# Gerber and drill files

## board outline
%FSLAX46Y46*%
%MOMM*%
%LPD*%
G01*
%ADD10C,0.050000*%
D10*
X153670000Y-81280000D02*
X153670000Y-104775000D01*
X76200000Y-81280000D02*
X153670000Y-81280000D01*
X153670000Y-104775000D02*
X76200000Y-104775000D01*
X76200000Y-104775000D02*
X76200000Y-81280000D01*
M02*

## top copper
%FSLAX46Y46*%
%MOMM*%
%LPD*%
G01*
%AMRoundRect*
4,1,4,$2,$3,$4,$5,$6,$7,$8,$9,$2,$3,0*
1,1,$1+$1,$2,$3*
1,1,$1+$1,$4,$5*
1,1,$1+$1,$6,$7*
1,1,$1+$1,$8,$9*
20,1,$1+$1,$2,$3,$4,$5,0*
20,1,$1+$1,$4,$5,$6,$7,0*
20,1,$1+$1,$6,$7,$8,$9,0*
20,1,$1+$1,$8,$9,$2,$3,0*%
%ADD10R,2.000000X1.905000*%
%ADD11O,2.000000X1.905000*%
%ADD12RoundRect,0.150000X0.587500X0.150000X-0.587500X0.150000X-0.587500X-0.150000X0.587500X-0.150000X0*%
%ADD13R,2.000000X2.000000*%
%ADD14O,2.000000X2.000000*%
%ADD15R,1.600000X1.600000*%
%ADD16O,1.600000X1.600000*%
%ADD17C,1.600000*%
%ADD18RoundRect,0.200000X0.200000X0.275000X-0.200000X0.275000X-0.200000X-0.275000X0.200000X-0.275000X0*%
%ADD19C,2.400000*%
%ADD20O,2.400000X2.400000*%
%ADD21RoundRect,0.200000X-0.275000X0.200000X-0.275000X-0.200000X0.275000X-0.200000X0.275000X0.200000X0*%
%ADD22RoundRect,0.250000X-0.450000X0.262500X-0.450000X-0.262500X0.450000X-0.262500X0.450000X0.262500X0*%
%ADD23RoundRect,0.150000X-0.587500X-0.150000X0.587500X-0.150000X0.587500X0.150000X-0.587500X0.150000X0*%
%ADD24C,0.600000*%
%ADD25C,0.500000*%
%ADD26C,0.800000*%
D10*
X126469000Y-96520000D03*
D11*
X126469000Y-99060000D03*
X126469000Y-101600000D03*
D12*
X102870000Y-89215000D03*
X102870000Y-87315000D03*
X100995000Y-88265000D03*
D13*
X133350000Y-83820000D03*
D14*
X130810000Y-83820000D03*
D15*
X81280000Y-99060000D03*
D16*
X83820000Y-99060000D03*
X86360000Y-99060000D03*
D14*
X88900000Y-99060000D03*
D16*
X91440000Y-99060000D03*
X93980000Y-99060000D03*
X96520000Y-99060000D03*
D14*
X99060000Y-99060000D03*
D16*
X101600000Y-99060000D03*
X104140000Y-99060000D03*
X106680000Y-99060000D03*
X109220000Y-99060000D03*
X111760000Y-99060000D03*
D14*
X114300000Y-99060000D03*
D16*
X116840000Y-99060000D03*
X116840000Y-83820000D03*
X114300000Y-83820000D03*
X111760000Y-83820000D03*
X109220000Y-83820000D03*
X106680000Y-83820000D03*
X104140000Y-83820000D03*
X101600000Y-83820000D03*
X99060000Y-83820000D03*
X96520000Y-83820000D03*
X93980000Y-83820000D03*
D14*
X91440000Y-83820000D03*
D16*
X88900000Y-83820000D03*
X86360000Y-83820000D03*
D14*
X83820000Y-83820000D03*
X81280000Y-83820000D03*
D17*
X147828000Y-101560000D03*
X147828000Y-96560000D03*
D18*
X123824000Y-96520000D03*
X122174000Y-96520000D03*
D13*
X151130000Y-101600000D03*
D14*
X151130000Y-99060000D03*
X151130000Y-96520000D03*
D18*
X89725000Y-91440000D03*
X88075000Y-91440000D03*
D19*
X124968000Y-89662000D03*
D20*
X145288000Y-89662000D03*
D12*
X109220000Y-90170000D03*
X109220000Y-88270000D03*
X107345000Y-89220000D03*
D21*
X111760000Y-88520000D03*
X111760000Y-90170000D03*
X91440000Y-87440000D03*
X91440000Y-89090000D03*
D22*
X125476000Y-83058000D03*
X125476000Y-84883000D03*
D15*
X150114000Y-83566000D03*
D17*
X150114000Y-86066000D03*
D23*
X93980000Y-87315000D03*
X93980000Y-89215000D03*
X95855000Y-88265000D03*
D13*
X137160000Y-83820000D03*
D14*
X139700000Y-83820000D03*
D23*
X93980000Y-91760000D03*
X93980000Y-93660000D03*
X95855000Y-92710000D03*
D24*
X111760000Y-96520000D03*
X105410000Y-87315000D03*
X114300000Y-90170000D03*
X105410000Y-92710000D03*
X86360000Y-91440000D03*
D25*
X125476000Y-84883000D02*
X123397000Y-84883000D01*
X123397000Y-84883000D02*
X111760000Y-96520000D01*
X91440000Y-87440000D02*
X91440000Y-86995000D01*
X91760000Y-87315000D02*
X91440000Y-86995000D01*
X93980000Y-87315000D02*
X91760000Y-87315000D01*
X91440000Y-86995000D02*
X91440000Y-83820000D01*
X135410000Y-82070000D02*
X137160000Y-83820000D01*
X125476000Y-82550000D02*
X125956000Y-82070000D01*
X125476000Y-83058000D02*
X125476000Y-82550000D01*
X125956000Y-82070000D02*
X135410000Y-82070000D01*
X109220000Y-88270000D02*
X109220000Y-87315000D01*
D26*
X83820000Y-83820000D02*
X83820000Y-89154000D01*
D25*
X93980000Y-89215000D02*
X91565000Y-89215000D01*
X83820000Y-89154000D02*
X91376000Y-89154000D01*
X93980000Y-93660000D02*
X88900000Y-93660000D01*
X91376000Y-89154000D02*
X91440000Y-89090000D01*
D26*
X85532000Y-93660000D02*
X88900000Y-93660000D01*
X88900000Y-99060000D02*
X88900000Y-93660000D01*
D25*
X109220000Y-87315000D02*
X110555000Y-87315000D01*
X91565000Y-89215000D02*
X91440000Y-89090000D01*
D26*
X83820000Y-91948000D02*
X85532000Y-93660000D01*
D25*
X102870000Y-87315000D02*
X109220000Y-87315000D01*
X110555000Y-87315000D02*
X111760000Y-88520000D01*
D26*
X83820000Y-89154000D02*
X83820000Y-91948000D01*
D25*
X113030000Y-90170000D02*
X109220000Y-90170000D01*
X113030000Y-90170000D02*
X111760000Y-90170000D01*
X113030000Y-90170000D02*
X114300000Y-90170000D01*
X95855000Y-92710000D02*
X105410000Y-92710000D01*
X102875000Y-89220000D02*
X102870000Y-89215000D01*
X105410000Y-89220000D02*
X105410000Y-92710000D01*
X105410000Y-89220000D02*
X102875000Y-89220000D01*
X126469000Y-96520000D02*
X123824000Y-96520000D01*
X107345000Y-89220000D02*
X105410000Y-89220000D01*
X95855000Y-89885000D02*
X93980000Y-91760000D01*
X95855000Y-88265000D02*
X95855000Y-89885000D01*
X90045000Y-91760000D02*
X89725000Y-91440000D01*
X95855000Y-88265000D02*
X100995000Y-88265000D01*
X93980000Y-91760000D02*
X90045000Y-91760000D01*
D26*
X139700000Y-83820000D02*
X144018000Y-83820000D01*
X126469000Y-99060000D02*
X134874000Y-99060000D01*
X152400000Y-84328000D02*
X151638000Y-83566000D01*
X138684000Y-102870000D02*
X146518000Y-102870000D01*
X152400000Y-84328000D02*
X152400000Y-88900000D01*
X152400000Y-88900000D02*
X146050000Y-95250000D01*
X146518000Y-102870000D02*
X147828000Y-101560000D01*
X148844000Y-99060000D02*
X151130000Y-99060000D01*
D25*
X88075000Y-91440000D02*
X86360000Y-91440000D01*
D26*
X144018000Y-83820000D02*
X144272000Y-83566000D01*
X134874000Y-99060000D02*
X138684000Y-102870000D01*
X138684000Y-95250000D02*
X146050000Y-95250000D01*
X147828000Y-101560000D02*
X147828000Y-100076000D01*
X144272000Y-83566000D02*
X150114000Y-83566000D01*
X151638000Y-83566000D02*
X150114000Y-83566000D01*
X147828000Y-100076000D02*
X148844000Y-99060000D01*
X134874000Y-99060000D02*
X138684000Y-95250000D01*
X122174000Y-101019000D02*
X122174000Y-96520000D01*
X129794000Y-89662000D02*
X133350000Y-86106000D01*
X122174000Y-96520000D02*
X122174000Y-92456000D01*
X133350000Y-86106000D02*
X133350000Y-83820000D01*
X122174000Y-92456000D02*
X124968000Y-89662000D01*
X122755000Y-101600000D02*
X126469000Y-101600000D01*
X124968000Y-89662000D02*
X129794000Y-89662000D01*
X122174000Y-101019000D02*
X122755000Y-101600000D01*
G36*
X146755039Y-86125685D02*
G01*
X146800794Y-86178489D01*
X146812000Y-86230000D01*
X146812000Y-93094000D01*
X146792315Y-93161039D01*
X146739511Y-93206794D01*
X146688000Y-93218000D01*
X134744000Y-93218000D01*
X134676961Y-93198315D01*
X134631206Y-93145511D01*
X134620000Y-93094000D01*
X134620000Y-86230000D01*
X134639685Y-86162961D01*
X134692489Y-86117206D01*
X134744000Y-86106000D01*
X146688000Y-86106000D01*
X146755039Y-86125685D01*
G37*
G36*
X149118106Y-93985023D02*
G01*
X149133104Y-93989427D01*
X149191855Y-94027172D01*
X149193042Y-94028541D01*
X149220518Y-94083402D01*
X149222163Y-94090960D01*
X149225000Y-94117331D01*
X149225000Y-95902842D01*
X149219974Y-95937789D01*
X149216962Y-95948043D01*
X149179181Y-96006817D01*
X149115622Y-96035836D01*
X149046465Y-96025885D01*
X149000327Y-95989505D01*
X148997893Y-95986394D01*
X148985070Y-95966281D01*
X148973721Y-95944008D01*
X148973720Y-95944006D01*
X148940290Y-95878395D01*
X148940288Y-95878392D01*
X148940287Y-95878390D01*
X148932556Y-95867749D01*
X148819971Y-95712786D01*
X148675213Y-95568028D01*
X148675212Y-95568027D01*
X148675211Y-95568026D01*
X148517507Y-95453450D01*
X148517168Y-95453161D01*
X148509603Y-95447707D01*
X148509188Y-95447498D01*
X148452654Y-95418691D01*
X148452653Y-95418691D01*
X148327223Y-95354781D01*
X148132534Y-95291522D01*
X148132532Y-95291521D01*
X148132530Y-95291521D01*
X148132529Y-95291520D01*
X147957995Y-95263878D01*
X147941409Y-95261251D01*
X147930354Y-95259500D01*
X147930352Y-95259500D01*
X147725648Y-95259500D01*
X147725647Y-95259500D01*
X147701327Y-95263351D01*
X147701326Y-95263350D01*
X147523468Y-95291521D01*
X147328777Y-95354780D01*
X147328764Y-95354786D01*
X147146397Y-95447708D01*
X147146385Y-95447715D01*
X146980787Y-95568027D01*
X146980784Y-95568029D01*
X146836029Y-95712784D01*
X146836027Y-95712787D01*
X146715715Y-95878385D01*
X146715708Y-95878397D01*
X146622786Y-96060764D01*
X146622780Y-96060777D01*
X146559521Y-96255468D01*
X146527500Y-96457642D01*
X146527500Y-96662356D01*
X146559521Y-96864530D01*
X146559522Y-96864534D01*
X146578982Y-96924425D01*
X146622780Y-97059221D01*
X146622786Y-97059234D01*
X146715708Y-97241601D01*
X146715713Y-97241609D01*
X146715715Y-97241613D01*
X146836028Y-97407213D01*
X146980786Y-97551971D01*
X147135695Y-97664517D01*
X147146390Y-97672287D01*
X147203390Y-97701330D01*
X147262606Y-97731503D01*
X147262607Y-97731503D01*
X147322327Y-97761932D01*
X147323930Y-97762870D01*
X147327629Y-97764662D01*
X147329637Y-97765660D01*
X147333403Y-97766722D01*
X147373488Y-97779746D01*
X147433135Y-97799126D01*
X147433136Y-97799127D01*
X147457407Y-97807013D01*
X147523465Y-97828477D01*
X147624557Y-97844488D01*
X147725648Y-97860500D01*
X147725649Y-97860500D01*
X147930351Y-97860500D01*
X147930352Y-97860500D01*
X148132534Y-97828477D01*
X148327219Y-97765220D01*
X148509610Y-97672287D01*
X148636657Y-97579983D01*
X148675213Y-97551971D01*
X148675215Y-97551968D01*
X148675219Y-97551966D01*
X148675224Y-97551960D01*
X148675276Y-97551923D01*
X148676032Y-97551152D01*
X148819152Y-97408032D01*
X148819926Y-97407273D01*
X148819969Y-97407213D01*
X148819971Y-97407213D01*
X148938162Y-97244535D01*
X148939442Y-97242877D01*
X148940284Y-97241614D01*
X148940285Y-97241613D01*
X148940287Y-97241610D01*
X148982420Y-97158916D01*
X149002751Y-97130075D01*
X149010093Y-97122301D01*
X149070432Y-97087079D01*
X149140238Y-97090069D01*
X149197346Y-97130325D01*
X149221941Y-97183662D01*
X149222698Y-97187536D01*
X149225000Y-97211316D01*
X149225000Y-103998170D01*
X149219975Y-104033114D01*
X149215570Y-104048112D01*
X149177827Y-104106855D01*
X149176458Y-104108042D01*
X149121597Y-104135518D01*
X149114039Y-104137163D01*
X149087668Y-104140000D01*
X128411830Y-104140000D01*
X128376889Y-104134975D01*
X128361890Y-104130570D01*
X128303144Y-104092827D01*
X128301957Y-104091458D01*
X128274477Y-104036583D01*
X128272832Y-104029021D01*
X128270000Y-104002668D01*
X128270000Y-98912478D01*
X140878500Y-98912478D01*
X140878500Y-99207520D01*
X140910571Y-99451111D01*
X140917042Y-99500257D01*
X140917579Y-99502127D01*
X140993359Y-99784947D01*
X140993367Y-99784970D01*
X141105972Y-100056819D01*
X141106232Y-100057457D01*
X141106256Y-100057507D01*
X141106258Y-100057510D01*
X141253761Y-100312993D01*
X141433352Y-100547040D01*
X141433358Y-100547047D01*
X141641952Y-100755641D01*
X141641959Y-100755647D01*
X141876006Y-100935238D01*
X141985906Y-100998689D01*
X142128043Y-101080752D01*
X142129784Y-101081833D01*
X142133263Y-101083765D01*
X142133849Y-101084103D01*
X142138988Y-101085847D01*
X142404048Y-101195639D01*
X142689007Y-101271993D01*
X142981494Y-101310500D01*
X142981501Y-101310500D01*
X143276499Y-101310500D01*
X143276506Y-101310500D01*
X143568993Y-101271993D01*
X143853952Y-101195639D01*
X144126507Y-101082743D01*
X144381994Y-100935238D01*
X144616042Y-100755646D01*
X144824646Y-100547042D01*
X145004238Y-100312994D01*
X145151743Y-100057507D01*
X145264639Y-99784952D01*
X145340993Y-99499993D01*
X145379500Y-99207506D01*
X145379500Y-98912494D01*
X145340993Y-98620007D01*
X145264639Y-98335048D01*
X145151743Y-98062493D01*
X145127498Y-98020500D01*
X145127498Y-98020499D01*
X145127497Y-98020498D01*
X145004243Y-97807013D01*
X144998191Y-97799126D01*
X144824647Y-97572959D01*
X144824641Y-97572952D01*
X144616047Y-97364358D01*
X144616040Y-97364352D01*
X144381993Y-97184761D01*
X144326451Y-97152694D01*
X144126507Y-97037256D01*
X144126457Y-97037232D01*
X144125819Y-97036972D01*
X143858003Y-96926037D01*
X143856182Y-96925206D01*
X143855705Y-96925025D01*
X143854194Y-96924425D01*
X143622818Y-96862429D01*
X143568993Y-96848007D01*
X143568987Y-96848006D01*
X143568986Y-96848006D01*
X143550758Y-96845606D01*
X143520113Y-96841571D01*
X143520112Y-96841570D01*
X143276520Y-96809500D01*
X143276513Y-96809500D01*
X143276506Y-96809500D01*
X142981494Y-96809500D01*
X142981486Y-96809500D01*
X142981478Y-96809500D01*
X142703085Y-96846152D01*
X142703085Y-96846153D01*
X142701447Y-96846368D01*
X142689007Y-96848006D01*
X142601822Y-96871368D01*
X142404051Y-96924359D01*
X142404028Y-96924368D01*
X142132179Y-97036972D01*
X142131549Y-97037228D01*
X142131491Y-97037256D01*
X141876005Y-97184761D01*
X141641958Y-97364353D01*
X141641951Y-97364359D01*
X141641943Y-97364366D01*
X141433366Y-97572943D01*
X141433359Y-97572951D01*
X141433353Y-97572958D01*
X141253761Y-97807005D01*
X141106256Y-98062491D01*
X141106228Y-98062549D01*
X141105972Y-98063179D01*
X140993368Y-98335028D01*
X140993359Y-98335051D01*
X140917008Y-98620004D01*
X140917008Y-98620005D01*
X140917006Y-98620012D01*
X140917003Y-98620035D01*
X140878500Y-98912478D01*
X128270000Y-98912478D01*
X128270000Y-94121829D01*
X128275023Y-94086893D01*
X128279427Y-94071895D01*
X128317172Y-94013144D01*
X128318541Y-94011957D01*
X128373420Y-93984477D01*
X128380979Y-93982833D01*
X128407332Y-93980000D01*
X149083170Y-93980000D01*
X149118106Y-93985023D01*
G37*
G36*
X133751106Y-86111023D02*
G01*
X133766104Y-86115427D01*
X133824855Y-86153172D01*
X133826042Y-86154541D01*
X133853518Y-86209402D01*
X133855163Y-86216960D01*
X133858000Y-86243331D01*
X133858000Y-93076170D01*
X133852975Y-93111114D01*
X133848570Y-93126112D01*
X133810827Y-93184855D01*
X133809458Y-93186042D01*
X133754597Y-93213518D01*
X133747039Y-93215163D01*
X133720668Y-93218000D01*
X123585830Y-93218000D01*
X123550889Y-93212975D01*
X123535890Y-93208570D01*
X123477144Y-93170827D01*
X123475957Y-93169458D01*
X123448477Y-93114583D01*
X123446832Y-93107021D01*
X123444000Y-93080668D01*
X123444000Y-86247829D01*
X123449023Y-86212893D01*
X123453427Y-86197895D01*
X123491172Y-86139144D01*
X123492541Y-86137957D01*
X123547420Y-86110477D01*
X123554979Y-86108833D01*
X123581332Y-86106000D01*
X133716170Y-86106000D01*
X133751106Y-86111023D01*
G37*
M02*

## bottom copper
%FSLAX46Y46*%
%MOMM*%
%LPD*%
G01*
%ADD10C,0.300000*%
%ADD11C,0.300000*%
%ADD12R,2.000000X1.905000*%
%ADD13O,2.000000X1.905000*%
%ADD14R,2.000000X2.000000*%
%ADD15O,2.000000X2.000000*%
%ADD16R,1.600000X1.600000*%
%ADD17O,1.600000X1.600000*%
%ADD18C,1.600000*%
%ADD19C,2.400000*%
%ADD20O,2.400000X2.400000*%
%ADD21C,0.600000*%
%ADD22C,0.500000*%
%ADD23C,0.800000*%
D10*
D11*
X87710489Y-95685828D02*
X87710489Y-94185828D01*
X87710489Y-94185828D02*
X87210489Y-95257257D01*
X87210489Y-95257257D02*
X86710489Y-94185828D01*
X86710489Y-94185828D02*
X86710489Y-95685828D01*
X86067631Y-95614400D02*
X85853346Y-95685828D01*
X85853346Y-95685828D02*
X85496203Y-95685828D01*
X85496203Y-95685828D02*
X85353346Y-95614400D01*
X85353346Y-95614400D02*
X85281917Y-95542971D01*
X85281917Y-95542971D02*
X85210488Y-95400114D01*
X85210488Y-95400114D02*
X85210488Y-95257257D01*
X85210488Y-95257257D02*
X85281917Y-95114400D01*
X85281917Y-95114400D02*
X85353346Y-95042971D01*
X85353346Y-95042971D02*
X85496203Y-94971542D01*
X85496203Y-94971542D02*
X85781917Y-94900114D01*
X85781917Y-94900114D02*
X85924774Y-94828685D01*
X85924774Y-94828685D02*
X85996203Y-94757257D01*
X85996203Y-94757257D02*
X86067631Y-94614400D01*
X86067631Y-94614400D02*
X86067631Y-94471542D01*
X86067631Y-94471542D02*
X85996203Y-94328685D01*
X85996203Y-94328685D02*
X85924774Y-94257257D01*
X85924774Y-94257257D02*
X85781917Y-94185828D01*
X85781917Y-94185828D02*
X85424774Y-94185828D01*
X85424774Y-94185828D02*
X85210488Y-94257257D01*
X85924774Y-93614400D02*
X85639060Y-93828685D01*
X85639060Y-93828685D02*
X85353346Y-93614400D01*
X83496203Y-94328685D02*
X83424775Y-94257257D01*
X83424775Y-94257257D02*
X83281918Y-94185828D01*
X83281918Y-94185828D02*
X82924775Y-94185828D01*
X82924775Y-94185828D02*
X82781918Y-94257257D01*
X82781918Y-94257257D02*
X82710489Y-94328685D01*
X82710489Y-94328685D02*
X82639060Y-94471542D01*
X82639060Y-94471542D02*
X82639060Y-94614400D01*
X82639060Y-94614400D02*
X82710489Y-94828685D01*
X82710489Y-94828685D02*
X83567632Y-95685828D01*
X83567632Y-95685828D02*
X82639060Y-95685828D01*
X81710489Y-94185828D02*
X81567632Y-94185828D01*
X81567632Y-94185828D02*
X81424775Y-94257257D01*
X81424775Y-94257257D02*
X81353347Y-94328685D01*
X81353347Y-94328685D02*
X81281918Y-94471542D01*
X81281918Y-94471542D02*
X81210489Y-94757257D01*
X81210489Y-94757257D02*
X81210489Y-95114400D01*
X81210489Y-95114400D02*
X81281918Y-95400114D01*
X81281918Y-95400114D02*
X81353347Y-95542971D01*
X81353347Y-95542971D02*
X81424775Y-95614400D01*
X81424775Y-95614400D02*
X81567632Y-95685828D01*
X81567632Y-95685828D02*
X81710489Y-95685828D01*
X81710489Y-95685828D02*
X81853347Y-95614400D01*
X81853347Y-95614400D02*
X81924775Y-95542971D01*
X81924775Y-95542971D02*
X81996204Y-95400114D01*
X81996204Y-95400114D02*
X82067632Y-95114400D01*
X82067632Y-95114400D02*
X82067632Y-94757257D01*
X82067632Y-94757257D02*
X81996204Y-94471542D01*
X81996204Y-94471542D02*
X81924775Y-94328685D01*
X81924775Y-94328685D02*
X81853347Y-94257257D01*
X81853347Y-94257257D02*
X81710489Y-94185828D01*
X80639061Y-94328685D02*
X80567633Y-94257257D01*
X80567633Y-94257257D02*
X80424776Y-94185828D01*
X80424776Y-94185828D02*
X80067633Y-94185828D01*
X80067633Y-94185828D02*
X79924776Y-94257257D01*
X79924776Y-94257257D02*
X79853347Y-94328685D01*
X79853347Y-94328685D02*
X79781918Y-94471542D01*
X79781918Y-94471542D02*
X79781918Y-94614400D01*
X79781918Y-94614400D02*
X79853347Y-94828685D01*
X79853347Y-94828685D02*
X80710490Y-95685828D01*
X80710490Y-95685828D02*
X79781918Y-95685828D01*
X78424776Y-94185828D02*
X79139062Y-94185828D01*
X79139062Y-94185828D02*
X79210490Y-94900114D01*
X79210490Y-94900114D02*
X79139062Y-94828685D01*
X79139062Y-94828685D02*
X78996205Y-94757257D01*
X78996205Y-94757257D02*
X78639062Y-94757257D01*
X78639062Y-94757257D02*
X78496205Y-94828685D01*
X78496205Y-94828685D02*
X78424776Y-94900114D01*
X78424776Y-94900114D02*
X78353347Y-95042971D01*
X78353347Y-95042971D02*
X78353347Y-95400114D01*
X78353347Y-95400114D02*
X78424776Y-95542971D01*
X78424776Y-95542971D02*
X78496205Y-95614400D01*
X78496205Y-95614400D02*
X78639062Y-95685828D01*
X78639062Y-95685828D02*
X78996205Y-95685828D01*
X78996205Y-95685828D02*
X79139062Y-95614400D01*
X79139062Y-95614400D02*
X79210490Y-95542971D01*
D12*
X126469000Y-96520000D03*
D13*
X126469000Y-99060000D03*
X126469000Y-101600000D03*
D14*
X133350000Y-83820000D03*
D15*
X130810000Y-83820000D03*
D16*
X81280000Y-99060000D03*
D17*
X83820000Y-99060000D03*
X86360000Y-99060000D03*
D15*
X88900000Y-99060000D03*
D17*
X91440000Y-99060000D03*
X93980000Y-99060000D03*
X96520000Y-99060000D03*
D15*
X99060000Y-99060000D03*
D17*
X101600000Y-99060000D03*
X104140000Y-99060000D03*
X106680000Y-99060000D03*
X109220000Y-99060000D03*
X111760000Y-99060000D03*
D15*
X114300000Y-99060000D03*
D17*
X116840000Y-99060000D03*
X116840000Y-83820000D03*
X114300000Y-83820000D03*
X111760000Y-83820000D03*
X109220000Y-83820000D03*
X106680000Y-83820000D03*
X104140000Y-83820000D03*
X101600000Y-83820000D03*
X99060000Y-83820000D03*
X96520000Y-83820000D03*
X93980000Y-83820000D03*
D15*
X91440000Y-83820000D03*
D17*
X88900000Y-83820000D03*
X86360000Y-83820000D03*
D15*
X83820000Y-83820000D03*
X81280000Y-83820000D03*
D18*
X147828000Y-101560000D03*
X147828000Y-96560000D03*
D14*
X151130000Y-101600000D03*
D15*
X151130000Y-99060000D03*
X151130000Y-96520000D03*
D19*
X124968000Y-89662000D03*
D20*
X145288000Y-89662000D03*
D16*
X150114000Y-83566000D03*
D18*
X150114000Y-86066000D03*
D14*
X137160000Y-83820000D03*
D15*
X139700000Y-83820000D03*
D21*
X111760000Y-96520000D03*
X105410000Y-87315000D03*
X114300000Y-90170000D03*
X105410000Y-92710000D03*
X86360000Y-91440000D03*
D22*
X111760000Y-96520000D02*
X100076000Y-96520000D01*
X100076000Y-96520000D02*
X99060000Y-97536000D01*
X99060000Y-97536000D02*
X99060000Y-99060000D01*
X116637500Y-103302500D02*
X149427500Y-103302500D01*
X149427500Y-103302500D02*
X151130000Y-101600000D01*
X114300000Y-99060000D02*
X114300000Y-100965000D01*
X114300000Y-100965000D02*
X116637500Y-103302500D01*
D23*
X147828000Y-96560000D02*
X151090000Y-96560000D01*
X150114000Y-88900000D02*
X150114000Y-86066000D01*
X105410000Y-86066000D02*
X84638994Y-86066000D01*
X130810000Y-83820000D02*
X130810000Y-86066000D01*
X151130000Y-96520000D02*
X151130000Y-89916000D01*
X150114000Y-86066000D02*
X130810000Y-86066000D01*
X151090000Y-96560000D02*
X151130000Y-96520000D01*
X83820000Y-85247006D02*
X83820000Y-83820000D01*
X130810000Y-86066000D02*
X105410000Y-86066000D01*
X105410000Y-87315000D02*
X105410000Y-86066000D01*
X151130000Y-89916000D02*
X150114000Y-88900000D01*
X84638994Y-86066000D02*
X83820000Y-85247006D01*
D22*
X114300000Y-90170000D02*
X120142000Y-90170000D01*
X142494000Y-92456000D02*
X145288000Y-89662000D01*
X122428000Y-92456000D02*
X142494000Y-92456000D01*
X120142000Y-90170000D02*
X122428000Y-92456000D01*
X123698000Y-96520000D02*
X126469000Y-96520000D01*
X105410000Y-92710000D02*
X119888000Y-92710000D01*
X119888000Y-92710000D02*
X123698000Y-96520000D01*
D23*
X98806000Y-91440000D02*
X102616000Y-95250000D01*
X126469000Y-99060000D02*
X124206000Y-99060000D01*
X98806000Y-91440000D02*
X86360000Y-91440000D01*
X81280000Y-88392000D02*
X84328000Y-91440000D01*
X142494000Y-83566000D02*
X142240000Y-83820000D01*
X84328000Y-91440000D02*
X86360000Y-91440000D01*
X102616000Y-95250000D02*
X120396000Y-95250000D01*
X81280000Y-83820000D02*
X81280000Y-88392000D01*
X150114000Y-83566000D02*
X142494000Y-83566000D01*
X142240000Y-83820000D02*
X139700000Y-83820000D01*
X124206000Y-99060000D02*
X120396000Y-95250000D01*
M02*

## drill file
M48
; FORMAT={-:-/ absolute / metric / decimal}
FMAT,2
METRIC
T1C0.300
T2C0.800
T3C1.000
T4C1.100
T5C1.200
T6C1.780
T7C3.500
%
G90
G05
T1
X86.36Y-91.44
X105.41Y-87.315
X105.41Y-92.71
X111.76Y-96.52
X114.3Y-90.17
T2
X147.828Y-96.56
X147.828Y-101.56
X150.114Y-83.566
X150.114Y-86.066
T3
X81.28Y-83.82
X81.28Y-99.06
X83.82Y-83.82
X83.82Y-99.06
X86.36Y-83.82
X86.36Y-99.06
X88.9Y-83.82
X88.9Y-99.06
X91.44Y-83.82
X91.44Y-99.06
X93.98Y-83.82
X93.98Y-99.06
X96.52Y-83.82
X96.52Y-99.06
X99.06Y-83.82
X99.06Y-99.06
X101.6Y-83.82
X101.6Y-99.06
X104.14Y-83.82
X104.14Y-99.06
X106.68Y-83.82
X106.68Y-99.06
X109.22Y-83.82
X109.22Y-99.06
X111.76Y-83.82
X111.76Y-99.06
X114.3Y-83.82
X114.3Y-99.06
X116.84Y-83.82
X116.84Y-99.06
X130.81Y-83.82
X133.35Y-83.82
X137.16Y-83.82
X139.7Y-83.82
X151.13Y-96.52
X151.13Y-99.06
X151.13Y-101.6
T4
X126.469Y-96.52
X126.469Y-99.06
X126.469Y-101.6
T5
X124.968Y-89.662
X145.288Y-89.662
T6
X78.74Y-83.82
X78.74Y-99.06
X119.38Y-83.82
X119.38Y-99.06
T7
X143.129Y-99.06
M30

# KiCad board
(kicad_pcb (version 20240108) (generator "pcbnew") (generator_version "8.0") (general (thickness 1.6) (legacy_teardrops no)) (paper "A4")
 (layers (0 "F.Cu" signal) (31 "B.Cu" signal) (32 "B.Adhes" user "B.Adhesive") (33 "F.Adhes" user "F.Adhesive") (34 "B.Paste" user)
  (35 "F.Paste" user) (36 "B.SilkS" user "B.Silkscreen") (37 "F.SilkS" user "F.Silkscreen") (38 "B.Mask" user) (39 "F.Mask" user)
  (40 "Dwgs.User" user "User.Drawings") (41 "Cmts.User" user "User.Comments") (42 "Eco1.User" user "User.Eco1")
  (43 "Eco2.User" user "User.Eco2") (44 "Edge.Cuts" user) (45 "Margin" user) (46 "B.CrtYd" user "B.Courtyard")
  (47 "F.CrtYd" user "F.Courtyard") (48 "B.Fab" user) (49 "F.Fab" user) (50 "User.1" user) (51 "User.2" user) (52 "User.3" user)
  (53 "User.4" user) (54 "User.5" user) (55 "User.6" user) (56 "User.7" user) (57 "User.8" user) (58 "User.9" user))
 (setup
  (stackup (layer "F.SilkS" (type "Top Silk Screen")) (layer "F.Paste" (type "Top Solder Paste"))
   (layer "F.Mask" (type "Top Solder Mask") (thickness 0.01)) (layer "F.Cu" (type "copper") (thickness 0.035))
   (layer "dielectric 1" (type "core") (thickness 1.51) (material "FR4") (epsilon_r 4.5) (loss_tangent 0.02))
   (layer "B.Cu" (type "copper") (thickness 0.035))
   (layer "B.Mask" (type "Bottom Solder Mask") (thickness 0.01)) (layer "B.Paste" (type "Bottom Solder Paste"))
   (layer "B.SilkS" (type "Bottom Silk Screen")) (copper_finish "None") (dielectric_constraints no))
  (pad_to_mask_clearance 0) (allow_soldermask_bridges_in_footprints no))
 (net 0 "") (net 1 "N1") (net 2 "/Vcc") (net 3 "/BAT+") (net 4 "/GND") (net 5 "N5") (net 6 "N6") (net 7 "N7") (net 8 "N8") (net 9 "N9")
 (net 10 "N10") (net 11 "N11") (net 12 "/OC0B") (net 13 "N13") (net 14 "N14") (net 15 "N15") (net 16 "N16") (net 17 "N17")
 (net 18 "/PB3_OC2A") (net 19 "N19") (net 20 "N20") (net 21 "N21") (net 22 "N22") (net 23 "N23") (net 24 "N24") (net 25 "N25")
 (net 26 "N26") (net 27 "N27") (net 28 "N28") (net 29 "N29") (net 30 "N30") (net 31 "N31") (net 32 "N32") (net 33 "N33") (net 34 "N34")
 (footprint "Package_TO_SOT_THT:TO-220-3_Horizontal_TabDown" (layer "F.Cu") (at 126.469 96.52 -90)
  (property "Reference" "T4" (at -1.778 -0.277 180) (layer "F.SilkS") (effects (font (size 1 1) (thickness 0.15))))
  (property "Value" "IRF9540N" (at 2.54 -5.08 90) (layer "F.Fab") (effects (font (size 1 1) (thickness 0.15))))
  (pad "" np_thru_hole oval (at 2.54 -16.66 270) (size 3.5 3.5) (drill 3.5) (layers "*.Cu" "*.Mask"))
  (pad "1" thru_hole rect (at 0 0 270) (size 1.905 2) (drill 1.1) (layers "*.Cu" "*.Mask") (remove_unused_layers no) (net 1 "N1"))
  (pad "2" thru_hole oval (at 2.54 0 270) (size 1.905 2) (drill 1.1) (layers "*.Cu" "*.Mask") (remove_unused_layers no) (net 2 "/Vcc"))
  (pad "3" thru_hole oval (at 5.08 0 270) (size 1.905 2) (drill 1.1) (layers "*.Cu" "*.Mask") (remove_unused_layers no) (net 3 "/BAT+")))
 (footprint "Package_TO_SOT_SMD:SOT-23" (layer "F.Cu") (at 101.9325 88.265 180)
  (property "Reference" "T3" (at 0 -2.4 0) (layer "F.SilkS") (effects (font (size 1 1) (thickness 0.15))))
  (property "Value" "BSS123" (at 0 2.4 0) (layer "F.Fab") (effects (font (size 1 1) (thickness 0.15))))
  (pad "1" smd roundrect (at -0.9375 -0.95 180) (size 1.475 0.6) (layers "F.Cu" "F.Paste" "F.Mask") (roundrect_rratio 0.25) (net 1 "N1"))
  (pad "2" smd roundrect (at -0.9375 0.95 180) (size 1.475 0.6) (layers "F.Cu" "F.Paste" "F.Mask") (roundrect_rratio 0.25) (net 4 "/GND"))
  (pad "3" smd roundrect (at 0.9375 0 180) (size 1.475 0.6) (layers "F.Cu" "F.Paste" "F.Mask") (roundrect_rratio 0.25) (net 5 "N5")))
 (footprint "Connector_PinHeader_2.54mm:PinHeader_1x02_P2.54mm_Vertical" (layer "F.Cu") (at 133.35 83.82 -90)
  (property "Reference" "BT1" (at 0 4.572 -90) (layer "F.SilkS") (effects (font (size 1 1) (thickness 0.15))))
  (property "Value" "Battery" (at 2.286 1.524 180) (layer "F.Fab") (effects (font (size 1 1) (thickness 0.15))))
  (pad "1" thru_hole rect (at 0 0 270) (size 2 2) (drill 1) (layers "*.Cu" "*.Mask") (remove_unused_layers no) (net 3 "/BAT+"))
  (pad "2" thru_hole oval (at 0 2.54 270) (size 2 2) (drill 1) (layers "*.Cu" "*.Mask") (remove_unused_layers no) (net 4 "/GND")))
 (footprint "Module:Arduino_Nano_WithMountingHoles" (layer "F.Cu") (at 81.28 99.06 90)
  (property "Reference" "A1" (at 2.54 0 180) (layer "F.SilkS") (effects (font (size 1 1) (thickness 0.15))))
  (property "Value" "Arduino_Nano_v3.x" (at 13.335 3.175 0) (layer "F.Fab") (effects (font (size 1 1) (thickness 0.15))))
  (pad "" np_thru_hole circle (at 0 -2.54 90) (size 1.78 1.78) (drill 1.78) (layers "*.Cu" "*.Mask"))
  (pad "" np_thru_hole circle (at 0 38.1 90) (size 1.78 1.78) (drill 1.78) (layers "*.Cu" "*.Mask"))
  (pad "" np_thru_hole circle (at 15.24 -2.54 90) (size 1.78 1.78) (drill 1.78) (layers "*.Cu" "*.Mask"))
  (pad "" np_thru_hole circle (at 15.24 38.1 90) (size 1.78 1.78) (drill 1.78) (layers "*.Cu" "*.Mask"))
  (pad "1" thru_hole rect (at 0 0 90) (size 1.6 1.6) (drill 1) (layers "*.Cu" "*.Mask") (remove_unused_layers no) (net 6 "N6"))
  (pad "2" thru_hole oval (at 0 2.54 90) (size 1.6 1.6) (drill 1) (layers "*.Cu" "*.Mask") (remove_unused_layers no) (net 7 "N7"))
  (pad "3" thru_hole oval (at 0 5.08 90) (size 1.6 1.6) (drill 1) (layers "*.Cu" "*.Mask") (remove_unused_layers no) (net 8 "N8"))
  (pad "4" thru_hole oval (at 0 7.62 90) (size 2 2) (drill 1) (layers "*.Cu" "*.Mask") (remove_unused_layers no) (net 4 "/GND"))
  (pad "5" thru_hole oval (at 0 10.16 90) (size 1.6 1.6) (drill 1) (layers "*.Cu" "*.Mask") (remove_unused_layers no) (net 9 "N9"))
  (pad "6" thru_hole oval (at 0 12.7 90) (size 1.6 1.6) (drill 1) (layers "*.Cu" "*.Mask") (remove_unused_layers no) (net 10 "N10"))
  (pad "7" thru_hole oval (at 0 15.24 90) (size 1.6 1.6) (drill 1) (layers "*.Cu" "*.Mask") (remove_unused_layers no) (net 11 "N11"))
  (pad "8" thru_hole oval (at 0 17.78 90) (size 2 2) (drill 1) (layers "*.Cu" "*.Mask") (remove_unused_layers no) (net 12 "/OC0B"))
  (pad "9" thru_hole oval (at 0 20.32 90) (size 1.6 1.6) (drill 1) (layers "*.Cu" "*.Mask") (remove_unused_layers no) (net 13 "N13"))
  (pad "10" thru_hole oval (at 0 22.86 90) (size 1.6 1.6) (drill 1) (layers "*.Cu" "*.Mask") (remove_unused_layers no) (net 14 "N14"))
  (pad "11" thru_hole oval (at 0 25.4 90) (size 1.6 1.6) (drill 1) (layers "*.Cu" "*.Mask") (remove_unused_layers no) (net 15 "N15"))
  (pad "12" thru_hole oval (at 0 27.94 90) (size 1.6 1.6) (drill 1) (layers "*.Cu" "*.Mask") (remove_unused_layers no) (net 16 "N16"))
  (pad "13" thru_hole oval (at 0 30.48 90) (size 1.6 1.6) (drill 1) (layers "*.Cu" "*.Mask") (remove_unused_layers no) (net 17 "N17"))
  (pad "14" thru_hole oval (at 0 33.02 90) (size 2 2) (drill 1) (layers "*.Cu" "*.Mask") (remove_unused_layers no) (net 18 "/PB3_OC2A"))
  (pad "15" thru_hole oval (at 0 35.56 90) (size 1.6 1.6) (drill 1) (layers "*.Cu" "*.Mask") (remove_unused_layers no) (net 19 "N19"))
  (pad "16" thru_hole oval (at 15.24 35.56 90) (size 1.6 1.6) (drill 1) (layers "*.Cu" "*.Mask") (remove_unused_layers no) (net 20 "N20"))
  (pad "17" thru_hole oval (at 15.24 33.02 90) (size 1.6 1.6) (drill 1) (layers "*.Cu" "*.Mask") (remove_unused_layers no) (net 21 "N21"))
  (pad "18" thru_hole oval (at 15.24 30.48 90) (size 1.6 1.6) (drill 1) (layers "*.Cu" "*.Mask") (remove_unused_layers no) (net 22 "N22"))
  (pad "19" thru_hole oval (at 15.24 27.94 90) (size 1.6 1.6) (drill 1) (layers "*.Cu" "*.Mask") (remove_unused_layers no) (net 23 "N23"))
  (pad "20" thru_hole oval (at 15.24 25.4 90) (size 1.6 1.6) (drill 1) (layers "*.Cu" "*.Mask") (remove_unused_layers no) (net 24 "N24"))
  (pad "21" thru_hole oval (at 15.24 22.86 90) (size 1.6 1.6) (drill 1) (layers "*.Cu" "*.Mask") (remove_unused_layers no) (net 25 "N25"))
  (pad "22" thru_hole oval (at 15.24 20.32 90) (size 1.6 1.6) (drill 1) (layers "*.Cu" "*.Mask") (remove_unused_layers no) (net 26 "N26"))
  (pad "23" thru_hole oval (at 15.24 17.78 90) (size 1.6 1.6) (drill 1) (layers "*.Cu" "*.Mask") (remove_unused_layers no) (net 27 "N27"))
  (pad "24" thru_hole oval (at 15.24 15.24 90) (size 1.6 1.6) (drill 1) (layers "*.Cu" "*.Mask") (remove_unused_layers no) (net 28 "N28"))
  (pad "25" thru_hole oval (at 15.24 12.7 90) (size 1.6 1.6) (drill 1) (layers "*.Cu" "*.Mask") (remove_unused_layers no) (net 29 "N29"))
  (pad "26" thru_hole oval (at 15.24 10.16 90) (size 2 2) (drill 1) (layers "*.Cu" "*.Mask") (remove_unused_layers no) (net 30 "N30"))
  (pad "27" thru_hole oval (at 15.24 7.62 90) (size 1.6 1.6) (drill 1) (layers "*.Cu" "*.Mask") (remove_unused_layers no) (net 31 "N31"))
  (pad "28" thru_hole oval (at 15.24 5.08 90) (size 1.6 1.6) (drill 1) (layers "*.Cu" "*.Mask") (remove_unused_layers no) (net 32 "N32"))
  (pad "29" thru_hole oval (at 15.24 2.54 90) (size 2 2) (drill 1) (layers "*.Cu" "*.Mask") (remove_unused_layers no) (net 4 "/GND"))
  (pad "30" thru_hole oval (at 15.24 0 90) (size 2 2) (drill 1) (layers "*.Cu" "*.Mask") (remove_unused_layers no) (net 2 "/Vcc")))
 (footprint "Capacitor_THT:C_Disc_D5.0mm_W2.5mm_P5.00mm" (layer "F.Cu") (at 147.828 101.56 90)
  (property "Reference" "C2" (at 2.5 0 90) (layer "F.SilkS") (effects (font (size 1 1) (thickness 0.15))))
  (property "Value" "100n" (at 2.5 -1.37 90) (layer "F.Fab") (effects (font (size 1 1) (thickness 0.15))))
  (pad "1" thru_hole circle (at 0 0 90) (size 1.6 1.6) (drill 0.8) (layers "*.Cu" "*.Mask") (remove_unused_layers no) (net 2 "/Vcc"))
  (pad "2" thru_hole circle (at 5 0 90) (size 1.6 1.6) (drill 0.8) (layers "*.Cu" "*.Mask") (remove_unused_layers no) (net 4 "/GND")))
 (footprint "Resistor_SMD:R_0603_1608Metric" (layer "F.Cu") (at 122.999 96.52 180)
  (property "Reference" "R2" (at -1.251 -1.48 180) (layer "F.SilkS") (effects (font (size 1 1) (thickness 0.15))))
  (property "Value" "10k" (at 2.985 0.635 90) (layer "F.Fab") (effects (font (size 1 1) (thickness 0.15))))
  (pad "1" smd roundrect (at -0.825 0 180) (size 0.8 0.95) (layers "F.Cu" "F.Paste" "F.Mask") (roundrect_rratio 0.25) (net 1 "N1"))
  (pad "2" smd roundrect (at 0.825 0 180) (size 0.8 0.95) (layers "F.Cu" "F.Paste" "F.Mask") (roundrect_rratio 0.25) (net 3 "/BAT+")))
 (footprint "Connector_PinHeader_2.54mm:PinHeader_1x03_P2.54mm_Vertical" (layer "F.Cu") (at 151.13 101.6 180)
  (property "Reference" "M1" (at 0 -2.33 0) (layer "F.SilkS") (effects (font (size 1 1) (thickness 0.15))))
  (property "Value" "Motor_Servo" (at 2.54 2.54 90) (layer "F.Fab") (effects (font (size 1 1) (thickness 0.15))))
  (pad "1" thru_hole rect (at 0 0 180) (size 2 2) (drill 1) (layers "*.Cu" "*.Mask") (remove_unused_layers no) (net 18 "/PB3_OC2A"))
  (pad "2" thru_hole oval (at 0 2.54 180) (size 2 2) (drill 1) (layers "*.Cu" "*.Mask") (remove_unused_layers no) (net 2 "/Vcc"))
  (pad "3" thru_hole oval (at 0 5.08 180) (size 2 2) (drill 1) (layers "*.Cu" "*.Mask") (remove_unused_layers no) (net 4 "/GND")))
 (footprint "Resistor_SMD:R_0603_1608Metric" (layer "F.Cu") (at 88.9 91.44 180)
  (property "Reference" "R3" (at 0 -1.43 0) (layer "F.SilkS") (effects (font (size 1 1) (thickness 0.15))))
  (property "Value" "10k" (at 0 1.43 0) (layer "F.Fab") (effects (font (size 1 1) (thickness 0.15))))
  (pad "1" smd roundrect (at -0.825 0 180) (size 0.8 0.95) (layers "F.Cu" "F.Paste" "F.Mask") (roundrect_rratio 0.25) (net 5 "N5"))
  (pad "2" smd roundrect (at 0.825 0 180) (size 0.8 0.95) (layers "F.Cu" "F.Paste" "F.Mask") (roundrect_rratio 0.25) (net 2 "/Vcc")))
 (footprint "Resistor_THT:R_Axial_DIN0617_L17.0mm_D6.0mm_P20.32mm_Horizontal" (layer "F.Cu") (at 124.968 89.662)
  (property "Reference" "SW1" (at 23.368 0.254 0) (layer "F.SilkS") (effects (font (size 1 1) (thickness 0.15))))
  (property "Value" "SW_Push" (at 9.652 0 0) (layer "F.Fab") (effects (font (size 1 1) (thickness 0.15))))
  (pad "1" thru_hole circle (at 0 0) (size 2.4 2.4) (drill 1.2) (layers "*.Cu" "*.Mask") (remove_unused_layers no) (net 3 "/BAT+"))
  (pad "2" thru_hole oval (at 20.32 0) (size 2.4 2.4) (drill 1.2) (layers "*.Cu" "*.Mask") (remove_unused_layers no) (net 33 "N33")))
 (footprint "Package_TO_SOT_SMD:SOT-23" (layer "F.Cu") (at 108.2825 89.22 180)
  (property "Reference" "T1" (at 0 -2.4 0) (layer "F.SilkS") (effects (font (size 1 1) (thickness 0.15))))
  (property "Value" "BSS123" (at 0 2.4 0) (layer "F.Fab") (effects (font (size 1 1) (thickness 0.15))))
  (pad "1" smd roundrect (at -0.9375 -0.95 180) (size 1.475 0.6) (layers "F.Cu" "F.Paste" "F.Mask") (roundrect_rratio 0.25) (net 33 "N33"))
  (pad "2" smd roundrect (at -0.9375 0.95 180) (size 1.475 0.6) (layers "F.Cu" "F.Paste" "F.Mask") (roundrect_rratio 0.25) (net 4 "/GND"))
  (pad "3" smd roundrect (at 0.9375 0 180) (size 1.475 0.6) (layers "F.Cu" "F.Paste" "F.Mask") (roundrect_rratio 0.25) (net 1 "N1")))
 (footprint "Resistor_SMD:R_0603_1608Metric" (layer "F.Cu") (at 111.76 89.345 -90)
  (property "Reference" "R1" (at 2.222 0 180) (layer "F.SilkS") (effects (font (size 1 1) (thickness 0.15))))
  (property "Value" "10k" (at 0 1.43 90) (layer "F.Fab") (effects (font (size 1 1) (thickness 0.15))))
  (pad "1" smd roundrect (at -0.825 0 270) (size 0.8 0.95) (layers "F.Cu" "F.Paste" "F.Mask") (roundrect_rratio 0.25) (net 4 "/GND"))
  (pad "2" smd roundrect (at 0.825 0 270) (size 0.8 0.95) (layers "F.Cu" "F.Paste" "F.Mask") (roundrect_rratio 0.25) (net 33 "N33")))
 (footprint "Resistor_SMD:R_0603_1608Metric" (layer "F.Cu") (at 91.44 88.265 -90)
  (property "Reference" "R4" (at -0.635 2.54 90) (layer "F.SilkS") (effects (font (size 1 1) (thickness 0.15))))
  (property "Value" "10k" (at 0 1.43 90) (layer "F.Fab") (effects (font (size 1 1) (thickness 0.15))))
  (pad "1" smd roundrect (at -0.825 0 270) (size 0.8 0.95) (layers "F.Cu" "F.Paste" "F.Mask") (roundrect_rratio 0.25) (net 30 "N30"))
  (pad "2" smd roundrect (at 0.825 0 270) (size 0.8 0.95) (layers "F.Cu" "F.Paste" "F.Mask") (roundrect_rratio 0.25) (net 4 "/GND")))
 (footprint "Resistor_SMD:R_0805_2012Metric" (layer "F.Cu") (at 125.476 83.9705 -90)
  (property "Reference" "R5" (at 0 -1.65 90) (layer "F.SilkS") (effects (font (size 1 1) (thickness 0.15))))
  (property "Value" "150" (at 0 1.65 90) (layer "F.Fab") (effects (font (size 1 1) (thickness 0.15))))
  (pad "1" smd roundrect (at -0.9125 0 270) (size 1.025 1.4) (layers "F.Cu" "F.Paste" "F.Mask") (roundrect_rratio 0.243902) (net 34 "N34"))
  (pad "2" smd roundrect (at 0.9125 0 270) (size 1.025 1.4) (layers "F.Cu" "F.Paste" "F.Mask") (roundrect_rratio 0.243902) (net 12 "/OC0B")))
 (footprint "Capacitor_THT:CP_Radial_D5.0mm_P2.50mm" (layer "F.Cu") (at 150.114 83.566 -90)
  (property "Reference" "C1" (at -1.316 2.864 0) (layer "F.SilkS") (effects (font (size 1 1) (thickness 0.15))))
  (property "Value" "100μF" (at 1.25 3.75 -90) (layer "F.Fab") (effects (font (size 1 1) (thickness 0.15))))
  (pad "1" thru_hole rect (at 0 0 270) (size 1.6 1.6) (drill 0.8) (layers "*.Cu" "*.Mask") (remove_unused_layers no) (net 2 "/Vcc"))
  (pad "2" thru_hole circle (at 2.5 0 270) (size 1.6 1.6) (drill 0.8) (layers "*.Cu" "*.Mask") (remove_unused_layers no) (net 4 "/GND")))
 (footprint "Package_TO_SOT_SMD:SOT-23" (layer "F.Cu") (at 94.9175 88.265)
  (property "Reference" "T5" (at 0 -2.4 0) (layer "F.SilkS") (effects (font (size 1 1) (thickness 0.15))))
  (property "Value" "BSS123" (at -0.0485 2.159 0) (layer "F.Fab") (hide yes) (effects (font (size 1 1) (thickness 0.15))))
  (pad "1" smd roundrect (at -0.9375 -0.95) (size 1.475 0.6) (layers "F.Cu" "F.Paste" "F.Mask") (roundrect_rratio 0.25) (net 30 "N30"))
  (pad "2" smd roundrect (at -0.9375 0.95) (size 1.475 0.6) (layers "F.Cu" "F.Paste" "F.Mask") (roundrect_rratio 0.25) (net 4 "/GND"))
  (pad "3" smd roundrect (at 0.9375 0) (size 1.475 0.6) (layers "F.Cu" "F.Paste" "F.Mask") (roundrect_rratio 0.25) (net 5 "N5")))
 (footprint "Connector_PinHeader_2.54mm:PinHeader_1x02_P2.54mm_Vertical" (layer "F.Cu") (at 137.16 83.82 90)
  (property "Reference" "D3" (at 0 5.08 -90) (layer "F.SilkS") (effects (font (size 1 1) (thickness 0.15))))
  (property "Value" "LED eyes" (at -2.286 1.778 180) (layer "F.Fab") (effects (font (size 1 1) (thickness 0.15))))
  (pad "1" thru_hole rect (at 0 0 90) (size 2 2) (drill 1) (layers "*.Cu" "*.Mask") (remove_unused_layers no) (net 34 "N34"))
  (pad "2" thru_hole oval (at 0 2.54 90) (size 2 2) (drill 1) (layers "*.Cu" "*.Mask") (remove_unused_layers no) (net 2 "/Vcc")))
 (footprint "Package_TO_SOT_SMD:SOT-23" (layer "F.Cu") (at 94.9175 92.71)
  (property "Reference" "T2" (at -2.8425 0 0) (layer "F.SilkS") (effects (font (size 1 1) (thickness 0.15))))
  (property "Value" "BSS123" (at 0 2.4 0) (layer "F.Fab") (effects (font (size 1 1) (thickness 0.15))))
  (pad "1" smd roundrect (at -0.9375 -0.95) (size 1.475 0.6) (layers "F.Cu" "F.Paste" "F.Mask") (roundrect_rratio 0.25) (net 5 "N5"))
  (pad "2" smd roundrect (at -0.9375 0.95) (size 1.475 0.6) (layers "F.Cu" "F.Paste" "F.Mask") (roundrect_rratio 0.25) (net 4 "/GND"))
  (pad "3" smd roundrect (at 0.9375 0) (size 1.475 0.6) (layers "F.Cu" "F.Paste" "F.Mask") (roundrect_rratio 0.25) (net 1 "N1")))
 (gr_line (start 153.67 81.28) (end 153.67 104.775) (stroke (width 0.05) (type default)) (layer "Edge.Cuts"))
 (gr_line (start 76.2 81.28) (end 153.67 81.28) (stroke (width 0.05) (type default)) (layer "Edge.Cuts"))
 (gr_line (start 153.67 104.775) (end 76.2 104.775) (stroke (width 0.05) (type default)) (layer "Edge.Cuts"))
 (gr_line (start 76.2 104.775) (end 76.2 81.28) (stroke (width 0.05) (type default)) (layer "Edge.Cuts"))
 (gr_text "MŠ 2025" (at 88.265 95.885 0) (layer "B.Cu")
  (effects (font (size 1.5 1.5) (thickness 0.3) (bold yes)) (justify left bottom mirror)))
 (segment (start 125.476 84.883) (end 123.397 84.883) (width 0.5) (layer "F.Cu") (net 12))
 (segment (start 123.397 84.883) (end 111.76 96.52) (width 0.5) (layer "F.Cu") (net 12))
 (via (at 111.76 96.52) (size 0.6) (drill 0.3) (layers "F.Cu" "B.Cu") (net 12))
 (segment (start 111.76 96.52) (end 100.076 96.52) (width 0.5) (layer "B.Cu") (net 12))
 (segment (start 100.076 96.52) (end 99.06 97.536) (width 0.5) (layer "B.Cu") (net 12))
 (segment (start 99.06 97.536) (end 99.06 99.06) (width 0.5) (layer "B.Cu") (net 12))
 (segment (start 116.6375 103.3025) (end 149.4275 103.3025) (width 0.5) (layer "B.Cu") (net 18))
 (segment (start 149.4275 103.3025) (end 151.13 101.6) (width 0.5) (layer "B.Cu") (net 18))
 (segment (start 114.3 99.06) (end 114.3 100.965) (width 0.5) (layer "B.Cu") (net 18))
 (segment (start 114.3 100.965) (end 116.6375 103.3025) (width 0.5) (layer "B.Cu") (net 18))
 (segment (start 91.44 87.44) (end 91.44 86.995) (width 0.5) (layer "F.Cu") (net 30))
 (segment (start 91.76 87.315) (end 91.44 86.995) (width 0.5) (layer "F.Cu") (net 30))
 (segment (start 93.98 87.315) (end 91.76 87.315) (width 0.5) (layer "F.Cu") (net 30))
 (segment (start 91.44 86.995) (end 91.44 83.82) (width 0.5) (layer "F.Cu") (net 30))
 (segment (start 135.41 82.07) (end 137.16 83.82) (width 0.5) (layer "F.Cu") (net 34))
 (segment (start 125.476 82.55) (end 125.956 82.07) (width 0.5) (layer "F.Cu") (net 34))
 (segment (start 125.476 83.058) (end 125.476 82.55) (width 0.5) (layer "F.Cu") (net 34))
 (segment (start 125.956 82.07) (end 135.41 82.07) (width 0.5) (layer "F.Cu") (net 34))
 (segment (start 109.22 88.27) (end 109.22 87.315) (width 0.5) (layer "F.Cu") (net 4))
 (segment (start 83.82 83.82) (end 83.82 89.154) (width 0.8) (layer "F.Cu") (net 4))
 (segment (start 93.98 89.215) (end 91.565 89.215) (width 0.5) (layer "F.Cu") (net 4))
 (segment (start 83.82 89.154) (end 91.376 89.154) (width 0.5) (layer "F.Cu") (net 4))
 (segment (start 93.98 93.66) (end 88.9 93.66) (width 0.5) (layer "F.Cu") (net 4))
 (segment (start 91.376 89.154) (end 91.44 89.09) (width 0.5) (layer "F.Cu") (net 4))
 (segment (start 85.532 93.66) (end 88.9 93.66) (width 0.8) (layer "F.Cu") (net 4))
 (segment (start 88.9 99.06) (end 88.9 93.66) (width 0.8) (layer "F.Cu") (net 4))
 (segment (start 109.22 87.315) (end 110.555 87.315) (width 0.5) (layer "F.Cu") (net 4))
 (segment (start 91.565 89.215) (end 91.44 89.09) (width 0.5) (layer "F.Cu") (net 4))
 (segment (start 83.82 91.948) (end 85.532 93.66) (width 0.8) (layer "F.Cu") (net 4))
 (segment (start 102.87 87.315) (end 109.22 87.315) (width 0.5) (layer "F.Cu") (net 4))
 (segment (start 110.555 87.315) (end 111.76 88.52) (width 0.5) (layer "F.Cu") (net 4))
 (segment (start 83.82 89.154) (end 83.82 91.948) (width 0.8) (layer "F.Cu") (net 4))
 (via (at 105.41 87.315) (size 0.6) (drill 0.3) (layers "F.Cu" "B.Cu") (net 4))
 (segment (start 147.828 96.56) (end 151.09 96.56) (width 0.8) (layer "B.Cu") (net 4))
 (segment (start 150.114 88.9) (end 150.114 86.066) (width 0.8) (layer "B.Cu") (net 4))
 (segment (start 105.41 86.066) (end 84.638994 86.066) (width 0.8) (layer "B.Cu") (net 4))
 (segment (start 130.81 83.82) (end 130.81 86.066) (width 0.8) (layer "B.Cu") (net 4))
 (segment (start 151.13 96.52) (end 151.13 89.916) (width 0.8) (layer "B.Cu") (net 4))
 (segment (start 150.114 86.066) (end 130.81 86.066) (width 0.8) (layer "B.Cu") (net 4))
 (segment (start 151.09 96.56) (end 151.13 96.52) (width 0.8) (layer "B.Cu") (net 4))
 (segment (start 83.82 85.247006) (end 83.82 83.82) (width 0.8) (layer "B.Cu") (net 4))
 (segment (start 130.81 86.066) (end 105.41 86.066) (width 0.8) (layer "B.Cu") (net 4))
 (segment (start 105.41 87.315) (end 105.41 86.066) (width 0.8) (layer "B.Cu") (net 4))
 (segment (start 151.13 89.916) (end 150.114 88.9) (width 0.8) (layer "B.Cu") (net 4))
 (segment (start 84.638994 86.066) (end 83.82 85.247006) (width 0.8) (layer "B.Cu") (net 4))
 (segment (start 113.03 90.17) (end 109.22 90.17) (width 0.5) (layer "F.Cu") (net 33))
 (segment (start 113.03 90.17) (end 111.76 90.17) (width 0.5) (layer "F.Cu") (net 33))
 (segment (start 113.03 90.17) (end 114.3 90.17) (width 0.5) (layer "F.Cu") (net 33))
 (via (at 114.3 90.17) (size 0.6) (drill 0.3) (layers "F.Cu" "B.Cu") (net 33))
 (segment (start 114.3 90.17) (end 120.142 90.17) (width 0.5) (layer "B.Cu") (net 33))
 (segment (start 142.494 92.456) (end 145.288 89.662) (width 0.5) (layer "B.Cu") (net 33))
 (segment (start 122.428 92.456) (end 142.494 92.456) (width 0.5) (layer "B.Cu") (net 33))
 (segment (start 120.142 90.17) (end 122.428 92.456) (width 0.5) (layer "B.Cu") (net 33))
 (segment (start 95.855 92.71) (end 105.41 92.71) (width 0.5) (layer "F.Cu") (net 1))
 (segment (start 102.875 89.22) (end 102.87 89.215) (width 0.5) (layer "F.Cu") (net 1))
 (segment (start 105.41 89.22) (end 105.41 92.71) (width 0.5) (layer "F.Cu") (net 1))
 (segment (start 105.41 89.22) (end 102.875 89.22) (width 0.5) (layer "F.Cu") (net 1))
 (segment (start 126.469 96.52) (end 123.824 96.52) (width 0.5) (layer "F.Cu") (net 1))
 (segment (start 107.345 89.22) (end 105.41 89.22) (width 0.5) (layer "F.Cu") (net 1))
 (via (at 105.41 92.71) (size 0.6) (drill 0.3) (layers "F.Cu" "B.Cu") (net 1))
 (segment (start 123.698 96.52) (end 126.469 96.52) (width 0.5) (layer "B.Cu") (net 1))
 (segment (start 105.41 92.71) (end 119.888 92.71) (width 0.5) (layer "B.Cu") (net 1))
 (segment (start 119.888 92.71) (end 123.698 96.52) (width 0.5) (layer "B.Cu") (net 1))
 (segment (start 95.855 89.885) (end 93.98 91.76) (width 0.5) (layer "F.Cu") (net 5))
 (segment (start 95.855 88.265) (end 95.855 89.885) (width 0.5) (layer "F.Cu") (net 5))
 (segment (start 90.045 91.76) (end 89.725 91.44) (width 0.5) (layer "F.Cu") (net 5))
 (segment (start 95.855 88.265) (end 100.995 88.265) (width 0.5) (layer "F.Cu") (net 5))
 (segment (start 93.98 91.76) (end 90.045 91.76) (width 0.5) (layer "F.Cu") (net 5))
 (segment (start 139.7 83.82) (end 144.018 83.82) (width 0.8) (layer "F.Cu") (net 2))
 (segment (start 126.469 99.06) (end 134.874 99.06) (width 0.8) (layer "F.Cu") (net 2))
 (segment (start 152.4 84.328) (end 151.638 83.566) (width 0.8) (layer "F.Cu") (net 2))
 (segment (start 138.684 102.87) (end 146.518 102.87) (width 0.8) (layer "F.Cu") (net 2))
 (segment (start 152.4 84.328) (end 152.4 88.9) (width 0.8) (layer "F.Cu") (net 2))
 (segment (start 152.4 88.9) (end 146.05 95.25) (width 0.8) (layer "F.Cu") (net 2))
 (segment (start 146.518 102.87) (end 147.828 101.56) (width 0.8) (layer "F.Cu") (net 2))
 (segment (start 148.844 99.06) (end 151.13 99.06) (width 0.8) (layer "F.Cu") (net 2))
 (segment (start 88.075 91.44) (end 86.36 91.44) (width 0.5) (layer "F.Cu") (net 2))
 (segment (start 144.018 83.82) (end 144.272 83.566) (width 0.8) (layer "F.Cu") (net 2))
 (segment (start 134.874 99.06) (end 138.684 102.87) (width 0.8) (layer "F.Cu") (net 2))
 (segment (start 138.684 95.25) (end 146.05 95.25) (width 0.8) (layer "F.Cu") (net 2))
 (segment (start 147.828 101.56) (end 147.828 100.076) (width 0.8) (layer "F.Cu") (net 2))
 (segment (start 144.272 83.566) (end 150.114 83.566) (width 0.8) (layer "F.Cu") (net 2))
 (segment (start 151.638 83.566) (end 150.114 83.566) (width 0.8) (layer "F.Cu") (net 2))
 (segment (start 147.828 100.076) (end 148.844 99.06) (width 0.8) (layer "F.Cu") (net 2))
 (segment (start 134.874 99.06) (end 138.684 95.25) (width 0.8) (layer "F.Cu") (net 2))
 (via (at 86.36 91.44) (size 0.6) (drill 0.3) (layers "F.Cu" "B.Cu") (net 2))
 (segment (start 98.806 91.44) (end 102.616 95.25) (width 0.8) (layer "B.Cu") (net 2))
 (segment (start 126.469 99.06) (end 124.206 99.06) (width 0.8) (layer "B.Cu") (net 2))
 (segment (start 98.806 91.44) (end 86.36 91.44) (width 0.8) (layer "B.Cu") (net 2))
 (segment (start 81.28 88.392) (end 84.328 91.44) (width 0.8) (layer "B.Cu") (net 2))
 (segment (start 142.494 83.566) (end 142.24 83.82) (width 0.8) (layer "B.Cu") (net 2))
 (segment (start 84.328 91.44) (end 86.36 91.44) (width 0.8) (layer "B.Cu") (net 2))
 (segment (start 102.616 95.25) (end 120.396 95.25) (width 0.8) (layer "B.Cu") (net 2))
 (segment (start 81.28 83.82) (end 81.28 88.392) (width 0.8) (layer "B.Cu") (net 2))
 (segment (start 150.114 83.566) (end 142.494 83.566) (width 0.8) (layer "B.Cu") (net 2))
 (segment (start 142.24 83.82) (end 139.7 83.82) (width 0.8) (layer "B.Cu") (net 2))
 (segment (start 124.206 99.06) (end 120.396 95.25) (width 0.8) (layer "B.Cu") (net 2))
 (segment (start 122.174 101.019) (end 122.174 96.52) (width 0.8) (layer "F.Cu") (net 3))
 (segment (start 129.794 89.662) (end 133.35 86.106) (width 0.8) (layer "F.Cu") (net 3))
 (segment (start 122.174 96.52) (end 122.174 92.456) (width 0.8) (layer "F.Cu") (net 3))
 (segment (start 133.35 86.106) (end 133.35 83.82) (width 0.8) (layer "F.Cu") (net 3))
 (segment (start 122.174 92.456) (end 124.968 89.662) (width 0.8) (layer "F.Cu") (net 3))
 (segment (start 122.755 101.6) (end 126.469 101.6) (width 0.8) (layer "F.Cu") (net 3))
 (segment (start 124.968 89.662) (end 129.794 89.662) (width 0.8) (layer "F.Cu") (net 3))
 (segment (start 122.174 101.019) (end 122.755 101.6) (width 0.8) (layer "F.Cu") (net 3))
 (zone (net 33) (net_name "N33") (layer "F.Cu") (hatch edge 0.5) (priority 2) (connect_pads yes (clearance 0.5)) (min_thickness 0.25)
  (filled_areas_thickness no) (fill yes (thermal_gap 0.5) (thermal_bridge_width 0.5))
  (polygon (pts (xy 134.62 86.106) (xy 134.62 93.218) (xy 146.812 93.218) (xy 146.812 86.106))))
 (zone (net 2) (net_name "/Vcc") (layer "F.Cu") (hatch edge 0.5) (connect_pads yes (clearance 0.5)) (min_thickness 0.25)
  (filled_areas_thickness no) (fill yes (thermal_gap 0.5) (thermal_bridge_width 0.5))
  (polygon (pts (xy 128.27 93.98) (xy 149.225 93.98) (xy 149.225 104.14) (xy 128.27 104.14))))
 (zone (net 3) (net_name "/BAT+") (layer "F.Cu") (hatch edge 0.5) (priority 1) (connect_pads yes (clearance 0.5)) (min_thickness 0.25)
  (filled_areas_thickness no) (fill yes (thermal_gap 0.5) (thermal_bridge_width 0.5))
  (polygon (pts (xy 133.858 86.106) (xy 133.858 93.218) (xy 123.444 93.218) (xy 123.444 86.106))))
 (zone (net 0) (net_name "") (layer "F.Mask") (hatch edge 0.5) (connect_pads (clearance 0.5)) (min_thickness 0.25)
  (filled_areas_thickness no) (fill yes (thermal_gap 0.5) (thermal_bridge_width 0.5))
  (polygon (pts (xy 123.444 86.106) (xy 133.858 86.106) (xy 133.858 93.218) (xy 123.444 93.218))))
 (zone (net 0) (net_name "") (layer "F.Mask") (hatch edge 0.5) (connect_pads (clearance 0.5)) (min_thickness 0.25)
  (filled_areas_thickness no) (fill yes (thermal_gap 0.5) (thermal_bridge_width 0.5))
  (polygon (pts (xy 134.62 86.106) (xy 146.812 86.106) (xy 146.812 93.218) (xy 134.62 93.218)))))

